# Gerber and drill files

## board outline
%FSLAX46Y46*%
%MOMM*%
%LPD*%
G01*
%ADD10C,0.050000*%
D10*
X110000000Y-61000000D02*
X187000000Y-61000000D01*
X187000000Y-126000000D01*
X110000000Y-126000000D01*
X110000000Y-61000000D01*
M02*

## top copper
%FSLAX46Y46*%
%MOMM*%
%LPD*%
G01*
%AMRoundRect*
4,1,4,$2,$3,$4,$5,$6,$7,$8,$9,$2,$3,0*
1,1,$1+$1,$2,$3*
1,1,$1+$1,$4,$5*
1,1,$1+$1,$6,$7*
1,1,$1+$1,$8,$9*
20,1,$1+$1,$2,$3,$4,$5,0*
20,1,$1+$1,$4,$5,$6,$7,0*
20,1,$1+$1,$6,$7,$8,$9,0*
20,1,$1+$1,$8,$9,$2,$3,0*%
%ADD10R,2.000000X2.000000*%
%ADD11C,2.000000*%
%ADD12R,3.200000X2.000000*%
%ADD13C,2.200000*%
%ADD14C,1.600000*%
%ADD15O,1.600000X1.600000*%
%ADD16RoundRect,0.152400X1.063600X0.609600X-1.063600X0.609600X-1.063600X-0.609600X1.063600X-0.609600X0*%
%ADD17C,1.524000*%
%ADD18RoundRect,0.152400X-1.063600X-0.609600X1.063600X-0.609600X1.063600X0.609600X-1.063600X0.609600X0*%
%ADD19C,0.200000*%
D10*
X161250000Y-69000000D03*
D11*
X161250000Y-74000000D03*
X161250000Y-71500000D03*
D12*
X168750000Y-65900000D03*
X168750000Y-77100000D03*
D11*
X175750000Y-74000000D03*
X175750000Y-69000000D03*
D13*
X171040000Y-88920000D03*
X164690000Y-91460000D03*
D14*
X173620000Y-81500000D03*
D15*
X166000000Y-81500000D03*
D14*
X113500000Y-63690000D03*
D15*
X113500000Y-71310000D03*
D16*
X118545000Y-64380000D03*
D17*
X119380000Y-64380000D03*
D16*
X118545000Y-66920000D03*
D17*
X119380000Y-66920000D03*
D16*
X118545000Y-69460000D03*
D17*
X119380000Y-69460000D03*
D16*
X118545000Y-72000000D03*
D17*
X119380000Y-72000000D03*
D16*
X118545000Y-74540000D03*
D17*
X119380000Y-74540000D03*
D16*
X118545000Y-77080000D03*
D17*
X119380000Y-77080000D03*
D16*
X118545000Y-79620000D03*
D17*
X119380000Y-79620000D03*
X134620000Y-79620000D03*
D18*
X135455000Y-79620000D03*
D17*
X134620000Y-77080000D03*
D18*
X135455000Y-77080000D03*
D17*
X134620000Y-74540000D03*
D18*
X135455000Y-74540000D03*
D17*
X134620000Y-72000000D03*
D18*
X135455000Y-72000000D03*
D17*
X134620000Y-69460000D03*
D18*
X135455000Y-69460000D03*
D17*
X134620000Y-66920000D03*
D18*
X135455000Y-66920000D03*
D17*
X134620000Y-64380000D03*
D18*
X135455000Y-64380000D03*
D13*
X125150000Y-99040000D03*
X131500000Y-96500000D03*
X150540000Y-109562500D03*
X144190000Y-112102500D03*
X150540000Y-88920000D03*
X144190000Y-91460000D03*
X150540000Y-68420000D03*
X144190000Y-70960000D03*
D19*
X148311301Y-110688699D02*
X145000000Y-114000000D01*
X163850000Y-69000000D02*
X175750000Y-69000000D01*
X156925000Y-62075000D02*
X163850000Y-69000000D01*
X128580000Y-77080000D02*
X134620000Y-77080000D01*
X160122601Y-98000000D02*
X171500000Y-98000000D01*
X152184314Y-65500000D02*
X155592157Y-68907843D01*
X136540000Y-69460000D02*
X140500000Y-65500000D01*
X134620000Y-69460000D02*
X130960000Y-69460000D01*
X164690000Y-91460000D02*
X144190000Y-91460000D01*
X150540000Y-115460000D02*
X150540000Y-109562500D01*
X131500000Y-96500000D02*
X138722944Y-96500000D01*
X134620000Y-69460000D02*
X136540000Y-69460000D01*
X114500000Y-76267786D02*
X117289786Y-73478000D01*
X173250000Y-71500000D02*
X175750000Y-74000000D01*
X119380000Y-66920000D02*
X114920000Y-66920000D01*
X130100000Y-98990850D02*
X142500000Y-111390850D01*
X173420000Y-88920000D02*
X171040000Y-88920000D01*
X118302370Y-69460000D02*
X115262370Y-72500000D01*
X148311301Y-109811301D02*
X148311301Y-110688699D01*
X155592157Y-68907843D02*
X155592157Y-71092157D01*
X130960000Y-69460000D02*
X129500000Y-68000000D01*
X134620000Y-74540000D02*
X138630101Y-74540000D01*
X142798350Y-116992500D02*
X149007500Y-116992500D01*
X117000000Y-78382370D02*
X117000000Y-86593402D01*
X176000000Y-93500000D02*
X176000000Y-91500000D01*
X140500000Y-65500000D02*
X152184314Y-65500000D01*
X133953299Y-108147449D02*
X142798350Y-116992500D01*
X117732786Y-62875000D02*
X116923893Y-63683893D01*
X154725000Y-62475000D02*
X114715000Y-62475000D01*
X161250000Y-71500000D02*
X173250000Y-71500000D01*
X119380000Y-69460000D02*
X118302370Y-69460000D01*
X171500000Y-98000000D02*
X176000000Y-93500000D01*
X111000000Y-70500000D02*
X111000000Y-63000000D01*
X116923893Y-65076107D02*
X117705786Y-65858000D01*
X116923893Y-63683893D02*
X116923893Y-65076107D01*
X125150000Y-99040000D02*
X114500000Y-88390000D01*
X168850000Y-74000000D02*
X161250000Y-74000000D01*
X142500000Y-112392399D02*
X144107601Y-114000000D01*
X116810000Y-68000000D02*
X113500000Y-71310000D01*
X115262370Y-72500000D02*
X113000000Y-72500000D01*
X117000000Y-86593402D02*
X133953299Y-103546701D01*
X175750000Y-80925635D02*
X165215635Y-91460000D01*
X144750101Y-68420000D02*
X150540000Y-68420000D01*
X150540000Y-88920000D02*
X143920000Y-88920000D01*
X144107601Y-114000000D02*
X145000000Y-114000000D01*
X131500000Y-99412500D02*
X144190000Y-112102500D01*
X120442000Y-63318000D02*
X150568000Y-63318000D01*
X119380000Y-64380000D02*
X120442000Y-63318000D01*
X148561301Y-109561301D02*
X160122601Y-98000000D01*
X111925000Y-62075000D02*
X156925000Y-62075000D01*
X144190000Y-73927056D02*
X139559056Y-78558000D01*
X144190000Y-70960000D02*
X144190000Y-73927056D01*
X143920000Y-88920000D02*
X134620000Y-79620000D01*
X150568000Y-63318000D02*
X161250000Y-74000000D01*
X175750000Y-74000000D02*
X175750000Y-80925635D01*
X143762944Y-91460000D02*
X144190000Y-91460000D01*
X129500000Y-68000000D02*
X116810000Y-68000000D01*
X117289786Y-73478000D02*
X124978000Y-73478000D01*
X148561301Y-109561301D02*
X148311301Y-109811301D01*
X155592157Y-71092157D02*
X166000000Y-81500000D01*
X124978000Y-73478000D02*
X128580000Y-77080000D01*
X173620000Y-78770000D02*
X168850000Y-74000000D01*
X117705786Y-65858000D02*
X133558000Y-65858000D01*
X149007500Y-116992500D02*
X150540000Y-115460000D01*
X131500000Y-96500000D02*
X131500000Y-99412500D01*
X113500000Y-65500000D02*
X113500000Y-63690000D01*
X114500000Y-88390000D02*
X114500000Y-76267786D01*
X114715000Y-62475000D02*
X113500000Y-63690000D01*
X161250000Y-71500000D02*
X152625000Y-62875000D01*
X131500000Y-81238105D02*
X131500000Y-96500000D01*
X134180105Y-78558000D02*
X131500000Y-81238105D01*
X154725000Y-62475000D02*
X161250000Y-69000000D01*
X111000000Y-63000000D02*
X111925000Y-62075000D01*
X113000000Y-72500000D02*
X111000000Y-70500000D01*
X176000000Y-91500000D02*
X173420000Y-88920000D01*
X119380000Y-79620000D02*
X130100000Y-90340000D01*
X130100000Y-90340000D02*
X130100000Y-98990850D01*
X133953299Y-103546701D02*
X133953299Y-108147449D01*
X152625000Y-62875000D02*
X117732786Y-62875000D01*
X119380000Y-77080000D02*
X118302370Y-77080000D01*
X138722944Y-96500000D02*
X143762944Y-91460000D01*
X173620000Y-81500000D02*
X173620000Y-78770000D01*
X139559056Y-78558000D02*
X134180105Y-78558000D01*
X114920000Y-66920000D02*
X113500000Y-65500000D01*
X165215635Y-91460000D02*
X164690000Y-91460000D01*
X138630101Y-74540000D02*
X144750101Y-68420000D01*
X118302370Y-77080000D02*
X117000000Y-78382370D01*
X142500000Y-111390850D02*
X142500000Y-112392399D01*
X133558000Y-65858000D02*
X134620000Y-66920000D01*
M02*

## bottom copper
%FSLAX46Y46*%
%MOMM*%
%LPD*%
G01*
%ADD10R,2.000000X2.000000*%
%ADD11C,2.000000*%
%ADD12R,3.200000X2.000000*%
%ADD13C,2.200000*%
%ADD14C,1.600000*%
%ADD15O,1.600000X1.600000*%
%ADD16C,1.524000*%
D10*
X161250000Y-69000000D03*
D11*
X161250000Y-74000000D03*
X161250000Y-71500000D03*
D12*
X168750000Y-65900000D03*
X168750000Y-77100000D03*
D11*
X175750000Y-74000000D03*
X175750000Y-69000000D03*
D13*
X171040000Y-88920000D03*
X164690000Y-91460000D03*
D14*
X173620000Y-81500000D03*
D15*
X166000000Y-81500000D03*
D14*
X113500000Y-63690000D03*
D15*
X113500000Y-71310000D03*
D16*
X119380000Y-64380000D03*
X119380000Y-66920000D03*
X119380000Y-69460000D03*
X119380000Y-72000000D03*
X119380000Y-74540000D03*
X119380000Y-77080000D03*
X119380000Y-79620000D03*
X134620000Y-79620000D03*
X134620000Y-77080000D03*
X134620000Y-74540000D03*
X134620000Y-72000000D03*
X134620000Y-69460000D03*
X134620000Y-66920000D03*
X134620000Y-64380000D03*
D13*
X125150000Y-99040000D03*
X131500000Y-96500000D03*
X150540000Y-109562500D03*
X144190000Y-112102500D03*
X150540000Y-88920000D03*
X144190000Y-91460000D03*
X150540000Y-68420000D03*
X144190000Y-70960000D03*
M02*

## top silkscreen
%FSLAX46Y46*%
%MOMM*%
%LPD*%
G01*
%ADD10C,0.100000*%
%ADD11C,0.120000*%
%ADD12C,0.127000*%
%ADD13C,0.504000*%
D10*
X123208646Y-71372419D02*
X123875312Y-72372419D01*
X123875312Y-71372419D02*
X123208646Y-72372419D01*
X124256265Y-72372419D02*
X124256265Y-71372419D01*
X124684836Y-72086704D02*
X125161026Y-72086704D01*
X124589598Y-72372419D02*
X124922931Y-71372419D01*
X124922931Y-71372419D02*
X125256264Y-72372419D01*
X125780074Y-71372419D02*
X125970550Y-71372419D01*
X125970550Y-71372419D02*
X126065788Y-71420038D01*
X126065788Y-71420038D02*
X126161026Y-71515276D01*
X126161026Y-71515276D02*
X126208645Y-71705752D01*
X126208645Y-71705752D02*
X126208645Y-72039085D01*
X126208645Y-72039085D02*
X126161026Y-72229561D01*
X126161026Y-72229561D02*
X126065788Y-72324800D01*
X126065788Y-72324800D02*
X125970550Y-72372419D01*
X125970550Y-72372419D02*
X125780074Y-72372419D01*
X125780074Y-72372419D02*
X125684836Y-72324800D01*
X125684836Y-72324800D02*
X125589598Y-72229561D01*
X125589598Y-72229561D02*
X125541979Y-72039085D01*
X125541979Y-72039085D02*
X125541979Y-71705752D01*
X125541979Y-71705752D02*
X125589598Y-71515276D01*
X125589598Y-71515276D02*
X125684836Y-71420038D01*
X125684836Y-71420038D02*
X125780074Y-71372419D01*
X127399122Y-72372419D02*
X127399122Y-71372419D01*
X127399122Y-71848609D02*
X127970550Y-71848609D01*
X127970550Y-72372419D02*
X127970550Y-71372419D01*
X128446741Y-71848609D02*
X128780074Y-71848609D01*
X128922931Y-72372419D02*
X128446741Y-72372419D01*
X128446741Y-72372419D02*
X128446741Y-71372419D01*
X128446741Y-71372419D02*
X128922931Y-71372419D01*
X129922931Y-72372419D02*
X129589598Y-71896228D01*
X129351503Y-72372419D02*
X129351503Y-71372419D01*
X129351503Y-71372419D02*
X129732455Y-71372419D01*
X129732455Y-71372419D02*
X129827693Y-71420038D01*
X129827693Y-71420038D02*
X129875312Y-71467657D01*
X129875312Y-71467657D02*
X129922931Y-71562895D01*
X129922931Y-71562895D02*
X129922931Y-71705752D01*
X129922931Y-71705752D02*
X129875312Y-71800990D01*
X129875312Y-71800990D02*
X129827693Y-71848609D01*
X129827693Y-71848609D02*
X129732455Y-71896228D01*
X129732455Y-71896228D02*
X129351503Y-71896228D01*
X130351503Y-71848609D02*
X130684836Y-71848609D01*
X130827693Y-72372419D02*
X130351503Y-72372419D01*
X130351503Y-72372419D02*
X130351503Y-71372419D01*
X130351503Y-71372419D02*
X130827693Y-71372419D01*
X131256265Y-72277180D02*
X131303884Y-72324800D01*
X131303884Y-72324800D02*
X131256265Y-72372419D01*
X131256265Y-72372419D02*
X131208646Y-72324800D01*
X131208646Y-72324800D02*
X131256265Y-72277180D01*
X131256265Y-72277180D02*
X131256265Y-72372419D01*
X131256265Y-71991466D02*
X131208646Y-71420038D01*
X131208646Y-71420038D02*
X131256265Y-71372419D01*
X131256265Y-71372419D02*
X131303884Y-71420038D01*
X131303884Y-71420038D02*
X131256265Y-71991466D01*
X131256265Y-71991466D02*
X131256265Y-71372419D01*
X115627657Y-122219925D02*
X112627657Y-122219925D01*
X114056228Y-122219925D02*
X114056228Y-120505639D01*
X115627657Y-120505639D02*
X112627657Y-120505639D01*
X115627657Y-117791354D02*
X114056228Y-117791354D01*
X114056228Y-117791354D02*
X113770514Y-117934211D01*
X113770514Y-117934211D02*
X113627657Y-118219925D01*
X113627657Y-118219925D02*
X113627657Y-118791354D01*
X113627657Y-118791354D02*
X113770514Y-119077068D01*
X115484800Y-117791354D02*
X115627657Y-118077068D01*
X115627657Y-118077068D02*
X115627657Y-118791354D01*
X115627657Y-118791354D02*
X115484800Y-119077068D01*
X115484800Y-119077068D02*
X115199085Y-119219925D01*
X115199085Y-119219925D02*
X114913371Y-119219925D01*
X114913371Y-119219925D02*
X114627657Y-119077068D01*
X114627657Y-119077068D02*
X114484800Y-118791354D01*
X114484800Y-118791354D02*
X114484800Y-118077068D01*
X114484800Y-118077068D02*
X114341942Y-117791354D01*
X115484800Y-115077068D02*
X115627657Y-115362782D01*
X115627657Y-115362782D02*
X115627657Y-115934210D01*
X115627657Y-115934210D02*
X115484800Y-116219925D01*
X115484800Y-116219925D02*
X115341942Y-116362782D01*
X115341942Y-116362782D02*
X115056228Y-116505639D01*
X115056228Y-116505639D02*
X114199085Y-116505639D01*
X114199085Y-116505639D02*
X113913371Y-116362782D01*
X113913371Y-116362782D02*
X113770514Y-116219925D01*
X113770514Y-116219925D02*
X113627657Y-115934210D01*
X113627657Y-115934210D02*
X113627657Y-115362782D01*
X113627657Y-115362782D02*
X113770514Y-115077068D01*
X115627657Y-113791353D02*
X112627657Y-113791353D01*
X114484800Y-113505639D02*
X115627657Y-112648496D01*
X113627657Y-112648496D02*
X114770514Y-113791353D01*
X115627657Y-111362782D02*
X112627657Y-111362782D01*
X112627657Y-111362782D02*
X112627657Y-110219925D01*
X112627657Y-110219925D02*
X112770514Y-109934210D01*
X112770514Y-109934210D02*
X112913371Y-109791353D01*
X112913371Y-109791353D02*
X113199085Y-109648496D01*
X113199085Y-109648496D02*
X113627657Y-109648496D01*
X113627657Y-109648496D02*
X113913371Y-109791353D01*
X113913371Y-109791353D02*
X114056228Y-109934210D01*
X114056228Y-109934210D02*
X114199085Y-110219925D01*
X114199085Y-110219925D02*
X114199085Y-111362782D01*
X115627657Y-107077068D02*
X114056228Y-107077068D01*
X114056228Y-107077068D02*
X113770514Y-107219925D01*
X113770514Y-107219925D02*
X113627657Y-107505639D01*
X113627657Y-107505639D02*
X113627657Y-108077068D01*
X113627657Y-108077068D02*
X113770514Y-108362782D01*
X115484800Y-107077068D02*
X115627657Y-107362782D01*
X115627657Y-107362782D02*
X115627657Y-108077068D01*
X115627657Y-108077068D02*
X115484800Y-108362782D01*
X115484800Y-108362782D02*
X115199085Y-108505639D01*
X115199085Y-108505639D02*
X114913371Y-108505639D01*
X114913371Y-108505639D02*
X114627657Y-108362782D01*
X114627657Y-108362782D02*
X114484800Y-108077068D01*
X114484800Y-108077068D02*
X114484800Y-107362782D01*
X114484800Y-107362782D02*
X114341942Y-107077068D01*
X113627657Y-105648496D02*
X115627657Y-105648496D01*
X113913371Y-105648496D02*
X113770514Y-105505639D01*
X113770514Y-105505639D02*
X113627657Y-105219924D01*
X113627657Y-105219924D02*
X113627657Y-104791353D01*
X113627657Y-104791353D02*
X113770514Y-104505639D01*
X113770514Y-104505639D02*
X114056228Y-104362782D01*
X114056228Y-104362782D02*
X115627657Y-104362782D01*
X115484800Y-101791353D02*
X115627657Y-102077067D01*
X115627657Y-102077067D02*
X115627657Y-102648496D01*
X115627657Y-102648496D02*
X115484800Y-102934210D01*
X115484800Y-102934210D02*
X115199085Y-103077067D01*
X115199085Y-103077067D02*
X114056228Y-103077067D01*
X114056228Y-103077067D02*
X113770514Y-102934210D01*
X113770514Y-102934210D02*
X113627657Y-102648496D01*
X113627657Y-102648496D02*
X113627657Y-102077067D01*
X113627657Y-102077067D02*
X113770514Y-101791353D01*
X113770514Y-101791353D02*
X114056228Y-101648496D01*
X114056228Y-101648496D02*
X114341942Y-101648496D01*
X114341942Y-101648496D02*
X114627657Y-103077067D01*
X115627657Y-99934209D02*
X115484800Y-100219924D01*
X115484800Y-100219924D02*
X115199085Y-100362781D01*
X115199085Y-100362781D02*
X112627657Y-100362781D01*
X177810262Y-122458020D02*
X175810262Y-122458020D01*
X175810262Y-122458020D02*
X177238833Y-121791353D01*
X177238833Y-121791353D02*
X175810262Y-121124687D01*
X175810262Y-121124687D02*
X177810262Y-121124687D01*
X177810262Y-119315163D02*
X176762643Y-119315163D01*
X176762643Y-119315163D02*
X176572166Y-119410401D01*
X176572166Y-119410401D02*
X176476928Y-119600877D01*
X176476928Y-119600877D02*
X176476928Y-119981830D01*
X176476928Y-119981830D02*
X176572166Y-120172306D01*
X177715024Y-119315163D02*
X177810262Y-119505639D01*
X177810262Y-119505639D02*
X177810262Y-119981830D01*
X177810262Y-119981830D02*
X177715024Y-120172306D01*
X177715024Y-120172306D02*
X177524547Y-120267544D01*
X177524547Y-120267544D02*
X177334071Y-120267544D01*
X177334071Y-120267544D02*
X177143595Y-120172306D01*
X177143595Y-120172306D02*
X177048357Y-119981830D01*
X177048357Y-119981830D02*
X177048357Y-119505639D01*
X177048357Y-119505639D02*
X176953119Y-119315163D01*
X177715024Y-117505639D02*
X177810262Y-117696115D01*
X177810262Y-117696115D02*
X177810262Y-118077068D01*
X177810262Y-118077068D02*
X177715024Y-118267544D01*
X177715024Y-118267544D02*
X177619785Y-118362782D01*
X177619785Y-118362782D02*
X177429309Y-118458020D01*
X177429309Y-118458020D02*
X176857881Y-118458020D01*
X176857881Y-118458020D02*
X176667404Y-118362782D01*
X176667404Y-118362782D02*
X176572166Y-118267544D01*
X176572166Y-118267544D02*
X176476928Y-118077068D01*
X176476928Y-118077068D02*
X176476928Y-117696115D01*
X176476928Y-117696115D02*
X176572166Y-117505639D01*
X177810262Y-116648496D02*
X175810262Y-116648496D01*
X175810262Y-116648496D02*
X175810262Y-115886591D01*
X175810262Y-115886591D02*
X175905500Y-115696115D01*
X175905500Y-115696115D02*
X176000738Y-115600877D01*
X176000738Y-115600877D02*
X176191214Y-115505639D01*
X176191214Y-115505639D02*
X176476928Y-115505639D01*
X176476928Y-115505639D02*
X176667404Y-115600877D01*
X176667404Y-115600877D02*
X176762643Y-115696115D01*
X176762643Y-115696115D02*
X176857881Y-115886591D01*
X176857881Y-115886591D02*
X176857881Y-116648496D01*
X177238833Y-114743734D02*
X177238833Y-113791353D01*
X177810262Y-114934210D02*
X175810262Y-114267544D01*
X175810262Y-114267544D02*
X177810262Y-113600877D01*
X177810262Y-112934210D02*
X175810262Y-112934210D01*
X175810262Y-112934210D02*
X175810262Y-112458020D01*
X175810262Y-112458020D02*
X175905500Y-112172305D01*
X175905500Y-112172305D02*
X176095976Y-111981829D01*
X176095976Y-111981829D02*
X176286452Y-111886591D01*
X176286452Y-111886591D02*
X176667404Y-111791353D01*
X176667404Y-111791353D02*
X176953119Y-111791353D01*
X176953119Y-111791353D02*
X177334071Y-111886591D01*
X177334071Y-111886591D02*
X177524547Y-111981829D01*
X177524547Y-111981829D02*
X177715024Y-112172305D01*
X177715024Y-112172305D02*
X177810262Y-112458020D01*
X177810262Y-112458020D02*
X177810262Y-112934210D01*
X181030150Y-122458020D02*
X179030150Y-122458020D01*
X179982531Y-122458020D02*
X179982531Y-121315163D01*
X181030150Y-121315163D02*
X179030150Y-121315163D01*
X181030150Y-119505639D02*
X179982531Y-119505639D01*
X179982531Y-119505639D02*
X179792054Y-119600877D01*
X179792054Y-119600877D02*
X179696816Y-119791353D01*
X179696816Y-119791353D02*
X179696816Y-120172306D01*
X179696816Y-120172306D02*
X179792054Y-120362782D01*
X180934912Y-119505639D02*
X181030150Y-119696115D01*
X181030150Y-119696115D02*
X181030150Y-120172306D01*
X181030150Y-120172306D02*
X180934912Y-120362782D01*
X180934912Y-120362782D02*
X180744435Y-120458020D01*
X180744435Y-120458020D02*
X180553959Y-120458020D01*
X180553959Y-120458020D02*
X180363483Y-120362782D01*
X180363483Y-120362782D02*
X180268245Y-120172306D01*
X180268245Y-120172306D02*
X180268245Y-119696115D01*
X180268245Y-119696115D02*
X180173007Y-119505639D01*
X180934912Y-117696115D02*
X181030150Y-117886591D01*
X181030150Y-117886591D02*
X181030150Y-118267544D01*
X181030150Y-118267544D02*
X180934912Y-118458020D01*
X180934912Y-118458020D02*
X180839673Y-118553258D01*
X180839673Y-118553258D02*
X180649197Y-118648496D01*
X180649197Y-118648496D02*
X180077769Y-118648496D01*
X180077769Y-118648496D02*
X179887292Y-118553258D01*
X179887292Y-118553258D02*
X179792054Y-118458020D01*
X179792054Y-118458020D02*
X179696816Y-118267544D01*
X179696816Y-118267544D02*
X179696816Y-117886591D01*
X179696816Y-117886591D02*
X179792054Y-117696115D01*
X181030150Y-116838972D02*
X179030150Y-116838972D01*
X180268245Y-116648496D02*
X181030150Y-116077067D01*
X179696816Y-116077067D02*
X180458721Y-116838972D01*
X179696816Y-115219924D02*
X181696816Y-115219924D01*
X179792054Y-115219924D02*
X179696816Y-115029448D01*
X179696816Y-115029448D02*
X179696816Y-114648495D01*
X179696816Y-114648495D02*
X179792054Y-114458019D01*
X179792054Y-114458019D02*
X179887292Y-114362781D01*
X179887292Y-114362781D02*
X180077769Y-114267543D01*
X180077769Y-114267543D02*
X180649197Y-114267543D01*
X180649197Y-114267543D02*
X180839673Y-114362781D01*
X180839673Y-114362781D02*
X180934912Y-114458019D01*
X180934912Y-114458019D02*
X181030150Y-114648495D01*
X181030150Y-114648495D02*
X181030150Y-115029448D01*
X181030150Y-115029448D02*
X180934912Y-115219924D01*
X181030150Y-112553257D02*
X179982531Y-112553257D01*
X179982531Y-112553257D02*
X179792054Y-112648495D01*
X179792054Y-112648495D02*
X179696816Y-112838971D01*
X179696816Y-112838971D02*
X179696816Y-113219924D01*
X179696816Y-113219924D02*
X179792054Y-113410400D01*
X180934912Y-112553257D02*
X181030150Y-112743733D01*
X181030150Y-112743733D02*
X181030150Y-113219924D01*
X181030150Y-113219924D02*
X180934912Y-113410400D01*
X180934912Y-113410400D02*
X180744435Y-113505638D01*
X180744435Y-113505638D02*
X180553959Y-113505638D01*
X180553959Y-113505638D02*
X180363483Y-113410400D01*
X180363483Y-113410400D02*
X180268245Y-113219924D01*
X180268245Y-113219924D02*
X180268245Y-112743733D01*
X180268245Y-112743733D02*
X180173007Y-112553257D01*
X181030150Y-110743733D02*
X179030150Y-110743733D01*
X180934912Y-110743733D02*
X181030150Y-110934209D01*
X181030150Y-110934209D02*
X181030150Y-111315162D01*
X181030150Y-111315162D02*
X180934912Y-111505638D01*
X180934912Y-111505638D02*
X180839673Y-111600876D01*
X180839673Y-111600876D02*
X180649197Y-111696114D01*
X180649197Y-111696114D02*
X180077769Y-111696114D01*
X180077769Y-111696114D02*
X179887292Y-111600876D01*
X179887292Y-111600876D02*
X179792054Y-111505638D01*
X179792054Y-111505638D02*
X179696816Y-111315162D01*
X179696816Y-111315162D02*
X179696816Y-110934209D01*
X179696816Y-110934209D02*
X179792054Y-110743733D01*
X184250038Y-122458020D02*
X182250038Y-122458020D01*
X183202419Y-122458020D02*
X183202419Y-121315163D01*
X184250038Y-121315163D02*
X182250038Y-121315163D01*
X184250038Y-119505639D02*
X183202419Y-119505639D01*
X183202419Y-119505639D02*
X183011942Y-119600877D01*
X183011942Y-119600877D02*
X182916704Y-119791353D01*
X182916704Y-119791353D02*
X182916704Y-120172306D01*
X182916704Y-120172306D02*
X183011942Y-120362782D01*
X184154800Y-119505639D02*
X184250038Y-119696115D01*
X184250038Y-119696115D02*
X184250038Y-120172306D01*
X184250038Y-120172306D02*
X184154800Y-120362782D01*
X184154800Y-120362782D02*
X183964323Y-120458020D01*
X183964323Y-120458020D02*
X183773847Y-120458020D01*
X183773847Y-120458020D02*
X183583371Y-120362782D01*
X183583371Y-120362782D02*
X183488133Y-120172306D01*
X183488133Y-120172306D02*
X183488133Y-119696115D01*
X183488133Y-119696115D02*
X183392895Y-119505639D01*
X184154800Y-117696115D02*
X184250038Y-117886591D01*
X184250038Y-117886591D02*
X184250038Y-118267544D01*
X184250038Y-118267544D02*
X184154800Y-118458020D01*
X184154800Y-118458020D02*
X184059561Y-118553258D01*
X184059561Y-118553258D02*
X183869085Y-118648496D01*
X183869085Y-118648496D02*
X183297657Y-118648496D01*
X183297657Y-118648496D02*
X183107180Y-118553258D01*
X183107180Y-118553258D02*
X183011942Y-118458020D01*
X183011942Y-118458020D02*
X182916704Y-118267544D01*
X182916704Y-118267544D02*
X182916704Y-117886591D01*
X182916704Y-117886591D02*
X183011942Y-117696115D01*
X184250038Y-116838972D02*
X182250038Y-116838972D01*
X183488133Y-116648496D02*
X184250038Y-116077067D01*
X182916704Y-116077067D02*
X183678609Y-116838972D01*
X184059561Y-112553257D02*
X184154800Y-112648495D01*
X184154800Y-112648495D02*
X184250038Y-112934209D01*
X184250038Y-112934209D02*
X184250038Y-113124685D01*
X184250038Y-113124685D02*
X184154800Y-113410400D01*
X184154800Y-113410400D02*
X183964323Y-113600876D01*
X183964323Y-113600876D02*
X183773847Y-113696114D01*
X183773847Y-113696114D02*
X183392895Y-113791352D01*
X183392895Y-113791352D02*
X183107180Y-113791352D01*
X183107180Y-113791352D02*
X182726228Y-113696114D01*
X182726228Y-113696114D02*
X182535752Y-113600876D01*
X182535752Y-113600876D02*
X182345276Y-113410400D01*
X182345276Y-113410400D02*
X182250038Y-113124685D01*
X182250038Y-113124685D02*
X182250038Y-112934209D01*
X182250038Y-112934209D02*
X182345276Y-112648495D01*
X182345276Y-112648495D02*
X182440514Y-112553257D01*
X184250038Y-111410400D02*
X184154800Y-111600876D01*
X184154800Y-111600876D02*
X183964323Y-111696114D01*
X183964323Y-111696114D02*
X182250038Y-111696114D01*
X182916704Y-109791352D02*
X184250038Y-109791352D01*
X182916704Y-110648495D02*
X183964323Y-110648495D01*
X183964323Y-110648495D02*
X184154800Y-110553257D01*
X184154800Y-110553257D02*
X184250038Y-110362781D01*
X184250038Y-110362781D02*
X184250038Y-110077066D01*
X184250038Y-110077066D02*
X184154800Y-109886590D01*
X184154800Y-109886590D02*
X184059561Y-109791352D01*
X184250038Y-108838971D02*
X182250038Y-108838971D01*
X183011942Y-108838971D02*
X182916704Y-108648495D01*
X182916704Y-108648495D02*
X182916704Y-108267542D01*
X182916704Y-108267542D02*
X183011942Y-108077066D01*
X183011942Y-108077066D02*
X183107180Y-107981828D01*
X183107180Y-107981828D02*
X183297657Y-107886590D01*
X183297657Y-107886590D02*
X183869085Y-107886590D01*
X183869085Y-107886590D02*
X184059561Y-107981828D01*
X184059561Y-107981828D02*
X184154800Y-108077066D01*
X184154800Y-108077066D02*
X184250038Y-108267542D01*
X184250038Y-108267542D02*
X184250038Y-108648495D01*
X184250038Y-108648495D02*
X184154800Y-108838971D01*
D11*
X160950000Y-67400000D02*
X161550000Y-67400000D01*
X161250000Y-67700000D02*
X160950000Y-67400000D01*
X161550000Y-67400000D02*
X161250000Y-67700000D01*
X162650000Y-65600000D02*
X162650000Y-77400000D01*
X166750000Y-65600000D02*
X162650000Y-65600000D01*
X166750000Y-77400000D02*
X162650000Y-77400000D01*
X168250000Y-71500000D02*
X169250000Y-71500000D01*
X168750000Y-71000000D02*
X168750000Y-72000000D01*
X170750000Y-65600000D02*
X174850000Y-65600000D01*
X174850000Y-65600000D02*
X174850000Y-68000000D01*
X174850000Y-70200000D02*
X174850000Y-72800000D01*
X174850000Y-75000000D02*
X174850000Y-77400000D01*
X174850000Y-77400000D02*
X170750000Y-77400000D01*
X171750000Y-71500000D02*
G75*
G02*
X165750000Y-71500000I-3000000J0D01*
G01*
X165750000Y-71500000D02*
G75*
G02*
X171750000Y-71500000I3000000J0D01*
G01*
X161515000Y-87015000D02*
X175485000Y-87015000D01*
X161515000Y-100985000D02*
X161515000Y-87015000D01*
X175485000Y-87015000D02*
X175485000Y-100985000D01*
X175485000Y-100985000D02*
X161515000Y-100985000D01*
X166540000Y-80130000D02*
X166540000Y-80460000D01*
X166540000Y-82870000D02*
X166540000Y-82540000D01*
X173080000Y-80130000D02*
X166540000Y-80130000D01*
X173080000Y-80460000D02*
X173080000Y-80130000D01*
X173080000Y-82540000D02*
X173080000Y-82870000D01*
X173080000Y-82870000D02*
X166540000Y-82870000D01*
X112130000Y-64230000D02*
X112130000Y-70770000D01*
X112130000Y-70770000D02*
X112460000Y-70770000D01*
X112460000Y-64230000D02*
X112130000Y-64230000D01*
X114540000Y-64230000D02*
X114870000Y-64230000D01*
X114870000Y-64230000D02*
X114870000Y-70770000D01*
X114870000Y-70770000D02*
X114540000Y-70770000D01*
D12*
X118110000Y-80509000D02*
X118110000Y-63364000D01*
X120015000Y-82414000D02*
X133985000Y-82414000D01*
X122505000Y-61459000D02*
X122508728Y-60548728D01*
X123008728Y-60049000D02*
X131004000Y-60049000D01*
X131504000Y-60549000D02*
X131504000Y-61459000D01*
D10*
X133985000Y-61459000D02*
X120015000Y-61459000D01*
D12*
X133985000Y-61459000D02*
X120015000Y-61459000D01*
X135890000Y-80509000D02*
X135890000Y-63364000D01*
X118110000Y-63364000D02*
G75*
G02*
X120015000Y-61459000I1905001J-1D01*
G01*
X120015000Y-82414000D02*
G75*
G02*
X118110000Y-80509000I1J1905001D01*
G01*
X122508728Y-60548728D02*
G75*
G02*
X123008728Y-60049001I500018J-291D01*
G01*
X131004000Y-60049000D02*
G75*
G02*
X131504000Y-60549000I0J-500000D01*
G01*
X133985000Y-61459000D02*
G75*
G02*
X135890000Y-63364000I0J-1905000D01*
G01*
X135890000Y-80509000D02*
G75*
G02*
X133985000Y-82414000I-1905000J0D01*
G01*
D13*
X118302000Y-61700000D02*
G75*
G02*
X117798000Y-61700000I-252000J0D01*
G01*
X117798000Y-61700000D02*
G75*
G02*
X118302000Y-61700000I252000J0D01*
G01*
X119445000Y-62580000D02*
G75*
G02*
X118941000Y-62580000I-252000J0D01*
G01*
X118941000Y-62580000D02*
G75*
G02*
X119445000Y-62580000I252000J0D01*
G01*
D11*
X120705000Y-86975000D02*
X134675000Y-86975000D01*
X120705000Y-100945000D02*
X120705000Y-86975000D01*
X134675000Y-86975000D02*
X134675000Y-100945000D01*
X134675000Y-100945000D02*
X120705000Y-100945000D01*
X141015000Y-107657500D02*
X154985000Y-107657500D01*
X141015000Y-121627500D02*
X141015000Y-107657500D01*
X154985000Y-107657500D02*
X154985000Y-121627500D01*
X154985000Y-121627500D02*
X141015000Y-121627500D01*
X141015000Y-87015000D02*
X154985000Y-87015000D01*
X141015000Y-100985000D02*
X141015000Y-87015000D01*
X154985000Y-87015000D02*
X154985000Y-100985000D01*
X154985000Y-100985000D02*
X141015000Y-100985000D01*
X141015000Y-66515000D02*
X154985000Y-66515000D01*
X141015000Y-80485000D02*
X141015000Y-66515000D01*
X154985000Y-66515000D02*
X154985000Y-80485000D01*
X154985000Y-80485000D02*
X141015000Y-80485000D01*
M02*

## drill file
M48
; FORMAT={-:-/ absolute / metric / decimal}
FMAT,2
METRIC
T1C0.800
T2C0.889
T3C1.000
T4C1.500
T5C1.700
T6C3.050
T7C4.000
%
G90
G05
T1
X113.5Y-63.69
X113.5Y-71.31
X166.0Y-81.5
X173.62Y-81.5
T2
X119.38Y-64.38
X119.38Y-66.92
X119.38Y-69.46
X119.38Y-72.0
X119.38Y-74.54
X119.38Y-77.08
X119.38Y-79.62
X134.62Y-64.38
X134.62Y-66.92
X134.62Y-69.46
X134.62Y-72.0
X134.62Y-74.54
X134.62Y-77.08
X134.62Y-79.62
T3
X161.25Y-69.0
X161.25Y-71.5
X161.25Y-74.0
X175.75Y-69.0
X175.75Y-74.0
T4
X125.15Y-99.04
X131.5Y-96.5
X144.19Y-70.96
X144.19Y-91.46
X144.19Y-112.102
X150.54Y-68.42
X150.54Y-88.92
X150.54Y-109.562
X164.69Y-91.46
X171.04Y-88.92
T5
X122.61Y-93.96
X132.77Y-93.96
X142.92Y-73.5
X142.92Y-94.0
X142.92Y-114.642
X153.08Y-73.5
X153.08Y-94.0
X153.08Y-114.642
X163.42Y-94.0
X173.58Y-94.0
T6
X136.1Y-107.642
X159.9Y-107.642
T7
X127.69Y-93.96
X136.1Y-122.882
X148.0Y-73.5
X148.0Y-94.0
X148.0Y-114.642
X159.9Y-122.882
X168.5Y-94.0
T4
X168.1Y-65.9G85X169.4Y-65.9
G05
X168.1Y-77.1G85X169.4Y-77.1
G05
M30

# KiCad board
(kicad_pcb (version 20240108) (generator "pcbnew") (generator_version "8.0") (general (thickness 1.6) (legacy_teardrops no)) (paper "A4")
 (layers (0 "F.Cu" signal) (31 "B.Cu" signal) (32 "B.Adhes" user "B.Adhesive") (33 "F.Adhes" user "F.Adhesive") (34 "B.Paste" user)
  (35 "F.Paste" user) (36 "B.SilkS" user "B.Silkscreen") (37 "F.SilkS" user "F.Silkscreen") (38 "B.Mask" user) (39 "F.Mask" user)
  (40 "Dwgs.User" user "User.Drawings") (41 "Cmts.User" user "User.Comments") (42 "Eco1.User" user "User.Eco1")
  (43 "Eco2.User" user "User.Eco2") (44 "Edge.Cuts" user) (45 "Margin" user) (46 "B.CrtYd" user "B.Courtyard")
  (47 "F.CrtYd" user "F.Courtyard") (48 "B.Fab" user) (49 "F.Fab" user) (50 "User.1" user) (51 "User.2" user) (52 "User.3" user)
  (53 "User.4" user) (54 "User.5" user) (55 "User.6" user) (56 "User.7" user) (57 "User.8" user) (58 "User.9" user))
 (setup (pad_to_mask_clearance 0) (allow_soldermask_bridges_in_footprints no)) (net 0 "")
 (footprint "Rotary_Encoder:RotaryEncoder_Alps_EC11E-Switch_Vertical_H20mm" (layer "F.Cu") (at 161.25 69)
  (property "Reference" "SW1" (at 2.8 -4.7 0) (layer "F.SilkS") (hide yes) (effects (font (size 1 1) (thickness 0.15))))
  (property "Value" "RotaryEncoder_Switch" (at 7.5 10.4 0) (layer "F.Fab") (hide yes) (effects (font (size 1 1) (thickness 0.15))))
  (fp_line (start -0.3 -1.6) (end 0.3 -1.6) (stroke (width 0.12) (type solid)) (layer "F.SilkS"))
  (fp_line (start 0 -1.3) (end -0.3 -1.6) (stroke (width 0.12) (type solid)) (layer "F.SilkS"))
  (fp_line (start 0.3 -1.6) (end 0 -1.3) (stroke (width 0.12) (type solid)) (layer "F.SilkS"))
  (fp_line (start 1.4 -3.4) (end 1.4 8.4) (stroke (width 0.12) (type solid)) (layer "F.SilkS"))
  (fp_line (start 5.5 -3.4) (end 1.4 -3.4) (stroke (width 0.12) (type solid)) (layer "F.SilkS"))
  (fp_line (start 5.5 8.4) (end 1.4 8.4) (stroke (width 0.12) (type solid)) (layer "F.SilkS"))
  (fp_line (start 7 2.5) (end 8 2.5) (stroke (width 0.12) (type solid)) (layer "F.SilkS"))
  (fp_line (start 7.5 2) (end 7.5 3) (stroke (width 0.12) (type solid)) (layer "F.SilkS"))
  (fp_line (start 9.5 -3.4) (end 13.6 -3.4) (stroke (width 0.12) (type solid)) (layer "F.SilkS"))
  (fp_line (start 13.6 -3.4) (end 13.6 -1) (stroke (width 0.12) (type solid)) (layer "F.SilkS"))
  (fp_line (start 13.6 1.2) (end 13.6 3.8) (stroke (width 0.12) (type solid)) (layer "F.SilkS"))
  (fp_line (start 13.6 6) (end 13.6 8.4) (stroke (width 0.12) (type solid)) (layer "F.SilkS"))
  (fp_line (start 13.6 8.4) (end 9.5 8.4) (stroke (width 0.12) (type solid)) (layer "F.SilkS"))
  (fp_circle (center 7.5 2.5) (end 10.5 2.5) (stroke (width 0.12) (type solid)) (fill none) (layer "F.SilkS"))
  (pad "A" thru_hole rect (at 0 0) (size 2 2) (drill 1) (layers "*.Cu" "*.Mask") (remove_unused_layers no))
  (pad "B" thru_hole circle (at 0 5) (size 2 2) (drill 1) (layers "*.Cu" "*.Mask") (remove_unused_layers no))
  (pad "C" thru_hole circle (at 0 2.5) (size 2 2) (drill 1) (layers "*.Cu" "*.Mask") (remove_unused_layers no))
  (pad "MP" thru_hole rect (at 7.5 -3.1) (size 3.2 2) (drill oval 2.8 1.5) (layers "*.Cu" "*.Mask") (remove_unused_layers no))
  (pad "MP" thru_hole rect (at 7.5 8.1) (size 3.2 2) (drill oval 2.8 1.5) (layers "*.Cu" "*.Mask") (remove_unused_layers no))
  (pad "S1" thru_hole circle (at 14.5 5) (size 2 2) (drill 1) (layers "*.Cu" "*.Mask") (remove_unused_layers no))
  (pad "S2" thru_hole circle (at 14.5 0) (size 2 2) (drill 1) (layers "*.Cu" "*.Mask") (remove_unused_layers no)))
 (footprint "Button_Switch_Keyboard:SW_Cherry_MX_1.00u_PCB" (layer "F.Cu") (at 171.04 88.92)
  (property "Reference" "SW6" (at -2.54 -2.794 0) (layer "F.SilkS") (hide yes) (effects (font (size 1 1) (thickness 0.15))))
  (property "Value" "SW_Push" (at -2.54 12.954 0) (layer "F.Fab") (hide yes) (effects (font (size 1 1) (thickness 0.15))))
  (fp_line (start -9.525 -1.905) (end 4.445 -1.905) (stroke (width 0.12) (type solid)) (layer "F.SilkS"))
  (fp_line (start -9.525 12.065) (end -9.525 -1.905) (stroke (width 0.12) (type solid)) (layer "F.SilkS"))
  (fp_line (start 4.445 -1.905) (end 4.445 12.065) (stroke (width 0.12) (type solid)) (layer "F.SilkS"))
  (fp_line (start 4.445 12.065) (end -9.525 12.065) (stroke (width 0.12) (type solid)) (layer "F.SilkS"))
  (pad "" np_thru_hole circle (at -7.62 5.08) (size 1.7 1.7) (drill 1.7) (layers "*.Cu" "*.Mask"))
  (pad "" np_thru_hole circle (at -2.54 5.08) (size 4 4) (drill 4) (layers "*.Cu" "*.Mask"))
  (pad "" np_thru_hole circle (at 2.54 5.08) (size 1.7 1.7) (drill 1.7) (layers "*.Cu" "*.Mask"))
  (pad "1" thru_hole circle (at 0 0) (size 2.2 2.2) (drill 1.5) (layers "*.Cu" "*.Mask") (remove_unused_layers no))
  (pad "2" thru_hole circle (at -6.35 2.54) (size 2.2 2.2) (drill 1.5) (layers "*.Cu" "*.Mask") (remove_unused_layers no)))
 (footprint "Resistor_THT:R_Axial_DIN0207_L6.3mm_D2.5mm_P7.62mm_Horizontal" (layer "F.Cu") (at 173.62 81.5 180)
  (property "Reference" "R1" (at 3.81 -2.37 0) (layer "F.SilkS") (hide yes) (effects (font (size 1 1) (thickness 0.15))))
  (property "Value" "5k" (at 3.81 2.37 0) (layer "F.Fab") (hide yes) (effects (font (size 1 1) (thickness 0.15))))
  (fp_line (start 7.08 1.37) (end 7.08 1.04) (stroke (width 0.12) (type solid)) (layer "F.SilkS"))
  (fp_line (start 7.08 -1.37) (end 7.08 -1.04) (stroke (width 0.12) (type solid)) (layer "F.SilkS"))
  (fp_line (start 0.54 1.37) (end 7.08 1.37) (stroke (width 0.12) (type solid)) (layer "F.SilkS"))
  (fp_line (start 0.54 1.04) (end 0.54 1.37) (stroke (width 0.12) (type solid)) (layer "F.SilkS"))
  (fp_line (start 0.54 -1.04) (end 0.54 -1.37) (stroke (width 0.12) (type solid)) (layer "F.SilkS"))
  (fp_line (start 0.54 -1.37) (end 7.08 -1.37) (stroke (width 0.12) (type solid)) (layer "F.SilkS"))
  (pad "1" thru_hole circle (at 0 0 180) (size 1.6 1.6) (drill 0.8) (layers "*.Cu" "*.Mask") (remove_unused_layers no))
  (pad "2" thru_hole oval (at 7.62 0 180) (size 1.6 1.6) (drill 0.8) (layers "*.Cu" "*.Mask") (remove_unused_layers no)))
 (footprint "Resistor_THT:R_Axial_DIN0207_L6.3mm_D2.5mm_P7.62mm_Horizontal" (layer "F.Cu") (at 113.5 63.69 -90)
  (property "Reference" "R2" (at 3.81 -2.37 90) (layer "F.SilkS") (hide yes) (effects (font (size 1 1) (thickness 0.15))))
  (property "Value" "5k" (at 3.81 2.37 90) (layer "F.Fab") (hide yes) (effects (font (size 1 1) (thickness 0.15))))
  (fp_line (start 0.54 1.37) (end 7.08 1.37) (stroke (width 0.12) (type solid)) (layer "F.SilkS"))
  (fp_line (start 7.08 1.37) (end 7.08 1.04) (stroke (width 0.12) (type solid)) (layer "F.SilkS"))
  (fp_line (start 0.54 1.04) (end 0.54 1.37) (stroke (width 0.12) (type solid)) (layer "F.SilkS"))
  (fp_line (start 0.54 -1.04) (end 0.54 -1.37) (stroke (width 0.12) (type solid)) (layer "F.SilkS"))
  (fp_line (start 0.54 -1.37) (end 7.08 -1.37) (stroke (width 0.12) (type solid)) (layer "F.SilkS"))
  (fp_line (start 7.08 -1.37) (end 7.08 -1.04) (stroke (width 0.12) (type solid)) (layer "F.SilkS"))
  (pad "1" thru_hole circle (at 0 0 270) (size 1.6 1.6) (drill 0.8) (layers "*.Cu" "*.Mask") (remove_unused_layers no))
  (pad "2" thru_hole oval (at 7.62 0 270) (size 1.6 1.6) (drill 0.8) (layers "*.Cu" "*.Mask") (remove_unused_layers no)))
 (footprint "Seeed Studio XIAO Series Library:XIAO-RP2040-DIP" (layer "F.Cu") (at 127 72)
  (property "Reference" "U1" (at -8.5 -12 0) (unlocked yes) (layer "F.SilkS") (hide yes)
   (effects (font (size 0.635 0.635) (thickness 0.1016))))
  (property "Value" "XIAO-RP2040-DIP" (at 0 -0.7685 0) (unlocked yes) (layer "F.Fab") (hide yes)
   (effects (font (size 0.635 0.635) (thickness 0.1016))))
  (fp_line (start -8.89 8.509) (end -8.89 -8.636) (stroke (width 0.127) (type solid)) (layer "F.SilkS"))
  (fp_line (start -6.985 10.414) (end 6.985 10.414) (stroke (width 0.127) (type solid)) (layer "F.SilkS"))
  (fp_line (start -4.495 -10.541) (end -4.491272 -11.451272) (stroke (width 0.127) (type solid)) (layer "F.SilkS"))
  (fp_line (start -3.991272 -11.951) (end 4.004 -11.951) (stroke (width 0.127) (type solid)) (layer "F.SilkS"))
  (fp_line (start 4.504 -11.451) (end 4.504 -10.541) (stroke (width 0.127) (type solid)) (layer "F.SilkS"))
  (fp_line (start 6.985 -10.541) (end -6.985 -10.541) (stroke (width 0.1) (type solid)) (layer "F.SilkS"))
  (fp_line (start 6.985 -10.541) (end -6.985 -10.541) (stroke (width 0.127) (type solid)) (layer "F.SilkS"))
  (fp_line (start 8.89 8.509) (end 8.89 -8.636) (stroke (width 0.127) (type solid)) (layer "F.SilkS"))
  (fp_arc (start -8.89 -8.636) (mid -8.332038 -9.983038) (end -6.985 -10.541) (stroke (width 0.127) (type solid)) (layer "F.SilkS"))
  (fp_arc (start -6.985 10.414) (mid -8.332038 9.856038) (end -8.89 8.509) (stroke (width 0.127) (type solid)) (layer "F.SilkS"))
  (fp_arc (start -4.491272 -11.451272) (mid -4.344724 -11.804644) (end -3.991272 -11.951) (stroke (width 0.127) (type default))
   (layer "F.SilkS"))
  (fp_arc (start 4.004 -11.951) (mid 4.357553 -11.804553) (end 4.504 -11.451) (stroke (width 0.127) (type default)) (layer "F.SilkS"))
  (fp_arc (start 6.985 -10.541) (mid 8.332038 -9.983038) (end 8.89 -8.636) (stroke (width 0.127) (type solid)) (layer "F.SilkS"))
  (fp_arc (start 8.89 8.509) (mid 8.332038 9.856038) (end 6.985 10.414) (stroke (width 0.127) (type solid)) (layer "F.SilkS"))
  (fp_circle (center -8.95 -10.3) (end -8.95 -10.554) (stroke (width 0.5) (type solid)) (fill solid) (layer "F.SilkS"))
  (fp_circle (center -7.807 -9.42) (end -7.807 -9.674) (stroke (width 0.5) (type solid)) (fill solid) (layer "F.SilkS"))
  (pad "1" smd roundrect (at -8.455 -7.62 180) (size 2.432 1.524) (layers "F.Cu" "F.Mask") (roundrect_rratio 0.1) (thermal_bridge_angle 45))
  (pad "1" thru_hole circle (at -7.62 -7.62 180) (size 1.524 1.524) (drill 0.889) (layers "*.Cu" "*.Mask") (remove_unused_layers no))
  (pad "2" smd roundrect (at -8.455 -5.08 180) (size 2.432 1.524) (layers "F.Cu" "F.Mask") (roundrect_rratio 0.1) (thermal_bridge_angle 45))
  (pad "2" thru_hole circle (at -7.62 -5.08 180) (size 1.524 1.524) (drill 0.889) (layers "*.Cu" "*.Mask") (remove_unused_layers no))
  (pad "3" smd roundrect (at -8.455 -2.54 180) (size 2.432 1.524) (layers "F.Cu" "F.Mask") (roundrect_rratio 0.1) (thermal_bridge_angle 45))
  (pad "3" thru_hole circle (at -7.62 -2.54 180) (size 1.524 1.524) (drill 0.889) (layers "*.Cu" "*.Mask") (remove_unused_layers no))
  (pad "4" smd roundrect (at -8.455 0 180) (size 2.432 1.524) (layers "F.Cu" "F.Mask") (roundrect_rratio 0.1) (thermal_bridge_angle 45))
  (pad "4" thru_hole circle (at -7.62 0 180) (size 1.524 1.524) (drill 0.889) (layers "*.Cu" "*.Mask") (remove_unused_layers no))
  (pad "5" smd roundrect (at -8.455 2.54 180) (size 2.432 1.524) (layers "F.Cu" "F.Mask") (roundrect_rratio 0.1) (thermal_bridge_angle 45))
  (pad "5" thru_hole circle (at -7.62 2.54 180) (size 1.524 1.524) (drill 0.889) (layers "*.Cu" "*.Mask") (remove_unused_layers no))
  (pad "6" smd roundrect (at -8.455 5.08 180) (size 2.432 1.524) (layers "F.Cu" "F.Mask") (roundrect_rratio 0.1) (thermal_bridge_angle 45))
  (pad "6" thru_hole circle (at -7.62 5.08 180) (size 1.524 1.524) (drill 0.889) (layers "*.Cu" "*.Mask") (remove_unused_layers no))
  (pad "7" smd roundrect (at -8.455 7.62 180) (size 2.432 1.524) (layers "F.Cu" "F.Mask") (roundrect_rratio 0.1) (thermal_bridge_angle 45))
  (pad "7" thru_hole circle (at -7.62 7.62 180) (size 1.524 1.524) (drill 0.889) (layers "*.Cu" "*.Mask") (remove_unused_layers no))
  (pad "8" thru_hole circle (at 7.62 7.62) (size 1.524 1.524) (drill 0.889) (layers "*.Cu" "*.Mask") (remove_unused_layers no))
  (pad "8" smd roundrect (at 8.455 7.62) (size 2.432 1.524) (layers "F.Cu" "F.Mask") (roundrect_rratio 0.1) (thermal_bridge_angle 45))
  (pad "9" thru_hole circle (at 7.62 5.08) (size 1.524 1.524) (drill 0.889) (layers "*.Cu" "*.Mask") (remove_unused_layers no))
  (pad "9" smd roundrect (at 8.455 5.08) (size 2.432 1.524) (layers "F.Cu" "F.Mask") (roundrect_rratio 0.1) (thermal_bridge_angle 45))
  (pad "10" thru_hole circle (at 7.62 2.54) (size 1.524 1.524) (drill 0.889) (layers "*.Cu" "*.Mask") (remove_unused_layers no))
  (pad "10" smd roundrect (at 8.455 2.54) (size 2.432 1.524) (layers "F.Cu" "F.Mask") (roundrect_rratio 0.1) (thermal_bridge_angle 45))
  (pad "11" thru_hole circle (at 7.62 0) (size 1.524 1.524) (drill 0.889) (layers "*.Cu" "*.Mask") (remove_unused_layers no))
  (pad "11" smd roundrect (at 8.455 0) (size 2.432 1.524) (layers "F.Cu" "F.Mask") (roundrect_rratio 0.1) (thermal_bridge_angle 45))
  (pad "12" thru_hole circle (at 7.62 -2.54) (size 1.524 1.524) (drill 0.889) (layers "*.Cu" "*.Mask") (remove_unused_layers no))
  (pad "12" smd roundrect (at 8.455 -2.54) (size 2.432 1.524) (layers "F.Cu" "F.Mask") (roundrect_rratio 0.1) (thermal_bridge_angle 45))
  (pad "13" thru_hole circle (at 7.62 -5.08) (size 1.524 1.524) (drill 0.889) (layers "*.Cu" "*.Mask") (remove_unused_layers no))
  (pad "13" smd roundrect (at 8.455 -5.08) (size 2.432 1.524) (layers "F.Cu" "F.Mask") (roundrect_rratio 0.1) (thermal_bridge_angle 45))
  (pad "14" thru_hole circle (at 7.62 -7.62) (size 1.524 1.524) (drill 0.889) (layers "*.Cu" "*.Mask") (remove_unused_layers no))
  (pad "14" smd roundrect (at 8.455 -7.62) (size 2.432 1.524) (layers "F.Cu" "F.Mask") (roundrect_rratio 0.1) (thermal_bridge_angle 45)))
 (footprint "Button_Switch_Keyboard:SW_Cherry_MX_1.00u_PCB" (layer "F.Cu") (at 125.15 99.04 180)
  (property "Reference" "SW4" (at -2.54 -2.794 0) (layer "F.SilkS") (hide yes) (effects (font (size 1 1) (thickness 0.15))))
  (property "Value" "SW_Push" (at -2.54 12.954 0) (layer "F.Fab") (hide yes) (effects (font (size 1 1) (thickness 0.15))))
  (fp_line (start 4.445 12.065) (end -9.525 12.065) (stroke (width 0.12) (type solid)) (layer "F.SilkS"))
  (fp_line (start 4.445 -1.905) (end 4.445 12.065) (stroke (width 0.12) (type solid)) (layer "F.SilkS"))
  (fp_line (start -9.525 12.065) (end -9.525 -1.905) (stroke (width 0.12) (type solid)) (layer "F.SilkS"))
  (fp_line (start -9.525 -1.905) (end 4.445 -1.905) (stroke (width 0.12) (type solid)) (layer "F.SilkS"))
  (pad "" np_thru_hole circle (at -7.62 5.08 180) (size 1.7 1.7) (drill 1.7) (layers "*.Cu" "*.Mask"))
  (pad "" np_thru_hole circle (at -2.54 5.08 180) (size 4 4) (drill 4) (layers "*.Cu" "*.Mask"))
  (pad "" np_thru_hole circle (at 2.54 5.08 180) (size 1.7 1.7) (drill 1.7) (layers "*.Cu" "*.Mask"))
  (pad "1" thru_hole circle (at 0 0 180) (size 2.2 2.2) (drill 1.5) (layers "*.Cu" "*.Mask") (remove_unused_layers no))
  (pad "2" thru_hole circle (at -6.35 2.54 180) (size 2.2 2.2) (drill 1.5) (layers "*.Cu" "*.Mask") (remove_unused_layers no)))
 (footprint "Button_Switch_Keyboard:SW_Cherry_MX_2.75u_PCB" (layer "F.Cu") (at 150.54 109.5625)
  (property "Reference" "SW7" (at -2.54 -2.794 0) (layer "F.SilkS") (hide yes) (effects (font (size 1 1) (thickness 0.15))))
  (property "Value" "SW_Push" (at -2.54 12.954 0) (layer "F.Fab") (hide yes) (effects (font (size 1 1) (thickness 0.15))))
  (fp_line (start -9.525 -1.905) (end 4.445 -1.905) (stroke (width 0.12) (type solid)) (layer "F.SilkS"))
  (fp_line (start -9.525 12.065) (end -9.525 -1.905) (stroke (width 0.12) (type solid)) (layer "F.SilkS"))
  (fp_line (start 4.445 -1.905) (end 4.445 12.065) (stroke (width 0.12) (type solid)) (layer "F.SilkS"))
  (fp_line (start 4.445 12.065) (end -9.525 12.065) (stroke (width 0.12) (type solid)) (layer "F.SilkS"))
  (pad "" np_thru_hole circle (at -14.44 -1.92) (size 3.05 3.05) (drill 3.05) (layers "*.Cu" "*.Mask"))
  (pad "" np_thru_hole circle (at -14.44 13.32) (size 4 4) (drill 4) (layers "*.Cu" "*.Mask"))
  (pad "" np_thru_hole circle (at -7.62 5.08) (size 1.7 1.7) (drill 1.7) (layers "*.Cu" "*.Mask"))
  (pad "" np_thru_hole circle (at -2.54 5.08) (size 4 4) (drill 4) (layers "*.Cu" "*.Mask"))
  (pad "" np_thru_hole circle (at 2.54 5.08) (size 1.7 1.7) (drill 1.7) (layers "*.Cu" "*.Mask"))
  (pad "" np_thru_hole circle (at 9.36 -1.92) (size 3.05 3.05) (drill 3.05) (layers "*.Cu" "*.Mask"))
  (pad "" np_thru_hole circle (at 9.36 13.32) (size 4 4) (drill 4) (layers "*.Cu" "*.Mask"))
  (pad "1" thru_hole circle (at 0 0) (size 2.2 2.2) (drill 1.5) (layers "*.Cu" "*.Mask") (remove_unused_layers no))
  (pad "2" thru_hole circle (at -6.35 2.54) (size 2.2 2.2) (drill 1.5) (layers "*.Cu" "*.Mask") (remove_unused_layers no)))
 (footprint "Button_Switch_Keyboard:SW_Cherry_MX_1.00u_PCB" (layer "F.Cu") (at 150.54 88.92)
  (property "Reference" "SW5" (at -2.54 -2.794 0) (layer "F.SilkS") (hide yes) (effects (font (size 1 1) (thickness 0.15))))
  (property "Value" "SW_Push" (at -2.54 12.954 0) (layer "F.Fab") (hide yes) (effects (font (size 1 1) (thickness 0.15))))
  (fp_line (start -9.525 -1.905) (end 4.445 -1.905) (stroke (width 0.12) (type solid)) (layer "F.SilkS"))
  (fp_line (start -9.525 12.065) (end -9.525 -1.905) (stroke (width 0.12) (type solid)) (layer "F.SilkS"))
  (fp_line (start 4.445 -1.905) (end 4.445 12.065) (stroke (width 0.12) (type solid)) (layer "F.SilkS"))
  (fp_line (start 4.445 12.065) (end -9.525 12.065) (stroke (width 0.12) (type solid)) (layer "F.SilkS"))
  (pad "" np_thru_hole circle (at -7.62 5.08) (size 1.7 1.7) (drill 1.7) (layers "*.Cu" "*.Mask"))
  (pad "" np_thru_hole circle (at -2.54 5.08) (size 4 4) (drill 4) (layers "*.Cu" "*.Mask"))
  (pad "" np_thru_hole circle (at 2.54 5.08) (size 1.7 1.7) (drill 1.7) (layers "*.Cu" "*.Mask"))
  (pad "1" thru_hole circle (at 0 0) (size 2.2 2.2) (drill 1.5) (layers "*.Cu" "*.Mask") (remove_unused_layers no))
  (pad "2" thru_hole circle (at -6.35 2.54) (size 2.2 2.2) (drill 1.5) (layers "*.Cu" "*.Mask") (remove_unused_layers no)))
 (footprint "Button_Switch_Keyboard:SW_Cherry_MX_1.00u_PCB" (layer "F.Cu") (at 150.54 68.42)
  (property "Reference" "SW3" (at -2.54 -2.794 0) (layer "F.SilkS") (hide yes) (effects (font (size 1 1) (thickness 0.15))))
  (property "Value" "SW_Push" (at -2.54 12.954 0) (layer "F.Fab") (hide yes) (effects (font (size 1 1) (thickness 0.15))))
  (fp_line (start -9.525 -1.905) (end 4.445 -1.905) (stroke (width 0.12) (type solid)) (layer "F.SilkS"))
  (fp_line (start -9.525 12.065) (end -9.525 -1.905) (stroke (width 0.12) (type solid)) (layer "F.SilkS"))
  (fp_line (start 4.445 -1.905) (end 4.445 12.065) (stroke (width 0.12) (type solid)) (layer "F.SilkS"))
  (fp_line (start 4.445 12.065) (end -9.525 12.065) (stroke (width 0.12) (type solid)) (layer "F.SilkS"))
  (pad "" np_thru_hole circle (at -7.62 5.08) (size 1.7 1.7) (drill 1.7) (layers "*.Cu" "*.Mask"))
  (pad "" np_thru_hole circle (at -2.54 5.08) (size 4 4) (drill 4) (layers "*.Cu" "*.Mask"))
  (pad "" np_thru_hole circle (at 2.54 5.08) (size 1.7 1.7) (drill 1.7) (layers "*.Cu" "*.Mask"))
  (pad "1" thru_hole circle (at 0 0) (size 2.2 2.2) (drill 1.5) (layers "*.Cu" "*.Mask") (remove_unused_layers no))
  (pad "2" thru_hole circle (at -6.35 2.54) (size 2.2 2.2) (drill 1.5) (layers "*.Cu" "*.Mask") (remove_unused_layers no)))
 (gr_rect (start 110 61) (end 187 126) (stroke (width 0.05) (type default)) (fill none) (layer "Edge.Cuts"))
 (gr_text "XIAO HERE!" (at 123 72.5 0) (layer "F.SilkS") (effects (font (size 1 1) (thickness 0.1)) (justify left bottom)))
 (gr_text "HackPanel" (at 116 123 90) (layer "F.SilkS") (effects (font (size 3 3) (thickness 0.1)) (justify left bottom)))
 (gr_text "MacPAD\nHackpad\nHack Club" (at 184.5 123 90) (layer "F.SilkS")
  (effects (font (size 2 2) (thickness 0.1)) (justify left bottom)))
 (segment (start 148.311301 110.688699) (end 145 114) (width 0.2) (layer "F.Cu") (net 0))
 (segment (start 163.85 69) (end 175.75 69) (width 0.2) (layer "F.Cu") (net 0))
 (segment (start 156.925 62.075) (end 163.85 69) (width 0.2) (layer "F.Cu") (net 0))
 (segment (start 128.58 77.08) (end 134.62 77.08) (width 0.2) (layer "F.Cu") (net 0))
 (segment (start 160.122601 98) (end 171.5 98) (width 0.2) (layer "F.Cu") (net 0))
 (segment (start 152.184314 65.5) (end 155.592157 68.907843) (width 0.2) (layer "F.Cu") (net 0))
 (segment (start 136.54 69.46) (end 140.5 65.5) (width 0.2) (layer "F.Cu") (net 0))
 (segment (start 134.62 69.46) (end 130.96 69.46) (width 0.2) (layer "F.Cu") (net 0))
 (segment (start 164.69 91.46) (end 144.19 91.46) (width 0.2) (layer "F.Cu") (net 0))
 (segment (start 150.54 115.46) (end 150.54 109.5625) (width 0.2) (layer "F.Cu") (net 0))
 (segment (start 131.5 96.5) (end 138.722944 96.5) (width 0.2) (layer "F.Cu") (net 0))
 (segment (start 134.62 69.46) (end 136.54 69.46) (width 0.2) (layer "F.Cu") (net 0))
 (segment (start 114.5 76.267786) (end 117.289786 73.478) (width 0.2) (layer "F.Cu") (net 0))
 (segment (start 173.25 71.5) (end 175.75 74) (width 0.2) (layer "F.Cu") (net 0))
 (segment (start 119.38 66.92) (end 114.92 66.92) (width 0.2) (layer "F.Cu") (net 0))
 (segment (start 130.1 98.99085) (end 142.5 111.39085) (width 0.2) (layer "F.Cu") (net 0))
 (segment (start 173.42 88.92) (end 171.04 88.92) (width 0.2) (layer "F.Cu") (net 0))
 (segment (start 118.30237 69.46) (end 115.26237 72.5) (width 0.2) (layer "F.Cu") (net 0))
 (segment (start 148.311301 109.811301) (end 148.311301 110.688699) (width 0.2) (layer "F.Cu") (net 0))
 (segment (start 155.592157 68.907843) (end 155.592157 71.092157) (width 0.2) (layer "F.Cu") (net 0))
 (segment (start 130.96 69.46) (end 129.5 68) (width 0.2) (layer "F.Cu") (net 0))
 (segment (start 134.62 74.54) (end 138.630101 74.54) (width 0.2) (layer "F.Cu") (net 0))
 (segment (start 142.79835 116.9925) (end 149.0075 116.9925) (width 0.2) (layer "F.Cu") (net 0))
 (segment (start 117 78.38237) (end 117 86.593402) (width 0.2) (layer "F.Cu") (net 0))
 (segment (start 176 93.5) (end 176 91.5) (width 0.2) (layer "F.Cu") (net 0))
 (segment (start 140.5 65.5) (end 152.184314 65.5) (width 0.2) (layer "F.Cu") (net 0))
 (segment (start 133.953299 108.147449) (end 142.79835 116.9925) (width 0.2) (layer "F.Cu") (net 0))
 (segment (start 117.732786 62.875) (end 116.923893 63.683893) (width 0.2) (layer "F.Cu") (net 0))
 (segment (start 154.725 62.475) (end 114.715 62.475) (width 0.2) (layer "F.Cu") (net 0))
 (segment (start 161.25 71.5) (end 173.25 71.5) (width 0.2) (layer "F.Cu") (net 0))
 (segment (start 119.38 69.46) (end 118.30237 69.46) (width 0.2) (layer "F.Cu") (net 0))
 (segment (start 171.5 98) (end 176 93.5) (width 0.2) (layer "F.Cu") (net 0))
 (segment (start 111 70.5) (end 111 63) (width 0.2) (layer "F.Cu") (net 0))
 (segment (start 116.923893 65.076107) (end 117.705786 65.858) (width 0.2) (layer "F.Cu") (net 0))
 (segment (start 116.923893 63.683893) (end 116.923893 65.076107) (width 0.2) (layer "F.Cu") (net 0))
 (segment (start 125.15 99.04) (end 114.5 88.39) (width 0.2) (layer "F.Cu") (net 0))
 (segment (start 168.85 74) (end 161.25 74) (width 0.2) (layer "F.Cu") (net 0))
 (segment (start 142.5 112.392399) (end 144.107601 114) (width 0.2) (layer "F.Cu") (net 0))
 (segment (start 116.81 68) (end 113.5 71.31) (width 0.2) (layer "F.Cu") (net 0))
 (segment (start 115.26237 72.5) (end 113 72.5) (width 0.2) (layer "F.Cu") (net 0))
 (segment (start 117 86.593402) (end 133.953299 103.546701) (width 0.2) (layer "F.Cu") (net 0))
 (segment (start 175.75 80.925635) (end 165.215635 91.46) (width 0.2) (layer "F.Cu") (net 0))
 (segment (start 144.750101 68.42) (end 150.54 68.42) (width 0.2) (layer "F.Cu") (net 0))
 (segment (start 150.54 88.92) (end 143.92 88.92) (width 0.2) (layer "F.Cu") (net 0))
 (segment (start 144.107601 114) (end 145 114) (width 0.2) (layer "F.Cu") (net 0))
 (segment (start 131.5 99.4125) (end 144.19 112.1025) (width 0.2) (layer "F.Cu") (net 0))
 (segment (start 120.442 63.318) (end 150.568 63.318) (width 0.2) (layer "F.Cu") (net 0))
 (segment (start 119.38 64.38) (end 120.442 63.318) (width 0.2) (layer "F.Cu") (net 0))
 (segment (start 148.561301 109.561301) (end 160.122601 98) (width 0.2) (layer "F.Cu") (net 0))
 (segment (start 111.925 62.075) (end 156.925 62.075) (width 0.2) (layer "F.Cu") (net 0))
 (segment (start 144.19 73.927056) (end 139.559056 78.558) (width 0.2) (layer "F.Cu") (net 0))
 (segment (start 144.19 70.96) (end 144.19 73.927056) (width 0.2) (layer "F.Cu") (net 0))
 (segment (start 143.92 88.92) (end 134.62 79.62) (width 0.2) (layer "F.Cu") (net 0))
 (segment (start 150.568 63.318) (end 161.25 74) (width 0.2) (layer "F.Cu") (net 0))
 (segment (start 175.75 74) (end 175.75 80.925635) (width 0.2) (layer "F.Cu") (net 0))
 (segment (start 143.762944 91.46) (end 144.19 91.46) (width 0.2) (layer "F.Cu") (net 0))
 (segment (start 129.5 68) (end 116.81 68) (width 0.2) (layer "F.Cu") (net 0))
 (segment (start 117.289786 73.478) (end 124.978 73.478) (width 0.2) (layer "F.Cu") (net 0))
 (segment (start 148.561301 109.561301) (end 148.311301 109.811301) (width 0.2) (layer "F.Cu") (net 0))
 (segment (start 155.592157 71.092157) (end 166 81.5) (width 0.2) (layer "F.Cu") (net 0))
 (segment (start 124.978 73.478) (end 128.58 77.08) (width 0.2) (layer "F.Cu") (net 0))
 (segment (start 173.62 78.77) (end 168.85 74) (width 0.2) (layer "F.Cu") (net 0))
 (segment (start 117.705786 65.858) (end 133.558 65.858) (width 0.2) (layer "F.Cu") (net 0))
 (segment (start 149.0075 116.9925) (end 150.54 115.46) (width 0.2) (layer "F.Cu") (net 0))
 (segment (start 131.5 96.5) (end 131.5 99.4125) (width 0.2) (layer "F.Cu") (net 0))
 (segment (start 113.5 65.5) (end 113.5 63.69) (width 0.2) (layer "F.Cu") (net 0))
 (segment (start 114.5 88.39) (end 114.5 76.267786) (width 0.2) (layer "F.Cu") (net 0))
 (segment (start 114.715 62.475) (end 113.5 63.69) (width 0.2) (layer "F.Cu") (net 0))
 (segment (start 161.25 71.5) (end 152.625 62.875) (width 0.2) (layer "F.Cu") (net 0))
 (segment (start 131.5 81.238105) (end 131.5 96.5) (width 0.2) (layer "F.Cu") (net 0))
 (segment (start 134.180105 78.558) (end 131.5 81.238105) (width 0.2) (layer "F.Cu") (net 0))
 (segment (start 154.725 62.475) (end 161.25 69) (width 0.2) (layer "F.Cu") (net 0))
 (segment (start 111 63) (end 111.925 62.075) (width 0.2) (layer "F.Cu") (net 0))
 (segment (start 113 72.5) (end 111 70.5) (width 0.2) (layer "F.Cu") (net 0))
 (segment (start 176 91.5) (end 173.42 88.92) (width 0.2) (layer "F.Cu") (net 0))
 (segment (start 119.38 79.62) (end 130.1 90.34) (width 0.2) (layer "F.Cu") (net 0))
 (segment (start 130.1 90.34) (end 130.1 98.99085) (width 0.2) (layer "F.Cu") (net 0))
 (segment (start 133.953299 103.546701) (end 133.953299 108.147449) (width 0.2) (layer "F.Cu") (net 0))
 (segment (start 152.625 62.875) (end 117.732786 62.875) (width 0.2) (layer "F.Cu") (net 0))
 (segment (start 119.38 77.08) (end 118.30237 77.08) (width 0.2) (layer "F.Cu") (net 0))
 (segment (start 138.722944 96.5) (end 143.762944 91.46) (width 0.2) (layer "F.Cu") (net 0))
 (segment (start 173.62 81.5) (end 173.62 78.77) (width 0.2) (layer "F.Cu") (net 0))
 (segment (start 139.559056 78.558) (end 134.180105 78.558) (width 0.2) (layer "F.Cu") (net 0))
 (segment (start 114.92 66.92) (end 113.5 65.5) (width 0.2) (layer "F.Cu") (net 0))
 (segment (start 165.215635 91.46) (end 164.69 91.46) (width 0.2) (layer "F.Cu") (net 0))
 (segment (start 138.630101 74.54) (end 144.750101 68.42) (width 0.2) (layer "F.Cu") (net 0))
 (segment (start 118.30237 77.08) (end 117 78.38237) (width 0.2) (layer "F.Cu") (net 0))
 (segment (start 142.5 111.39085) (end 142.5 112.392399) (width 0.2) (layer "F.Cu") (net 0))
 (segment (start 133.558 65.858) (end 134.62 66.92) (width 0.2) (layer "F.Cu") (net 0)))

